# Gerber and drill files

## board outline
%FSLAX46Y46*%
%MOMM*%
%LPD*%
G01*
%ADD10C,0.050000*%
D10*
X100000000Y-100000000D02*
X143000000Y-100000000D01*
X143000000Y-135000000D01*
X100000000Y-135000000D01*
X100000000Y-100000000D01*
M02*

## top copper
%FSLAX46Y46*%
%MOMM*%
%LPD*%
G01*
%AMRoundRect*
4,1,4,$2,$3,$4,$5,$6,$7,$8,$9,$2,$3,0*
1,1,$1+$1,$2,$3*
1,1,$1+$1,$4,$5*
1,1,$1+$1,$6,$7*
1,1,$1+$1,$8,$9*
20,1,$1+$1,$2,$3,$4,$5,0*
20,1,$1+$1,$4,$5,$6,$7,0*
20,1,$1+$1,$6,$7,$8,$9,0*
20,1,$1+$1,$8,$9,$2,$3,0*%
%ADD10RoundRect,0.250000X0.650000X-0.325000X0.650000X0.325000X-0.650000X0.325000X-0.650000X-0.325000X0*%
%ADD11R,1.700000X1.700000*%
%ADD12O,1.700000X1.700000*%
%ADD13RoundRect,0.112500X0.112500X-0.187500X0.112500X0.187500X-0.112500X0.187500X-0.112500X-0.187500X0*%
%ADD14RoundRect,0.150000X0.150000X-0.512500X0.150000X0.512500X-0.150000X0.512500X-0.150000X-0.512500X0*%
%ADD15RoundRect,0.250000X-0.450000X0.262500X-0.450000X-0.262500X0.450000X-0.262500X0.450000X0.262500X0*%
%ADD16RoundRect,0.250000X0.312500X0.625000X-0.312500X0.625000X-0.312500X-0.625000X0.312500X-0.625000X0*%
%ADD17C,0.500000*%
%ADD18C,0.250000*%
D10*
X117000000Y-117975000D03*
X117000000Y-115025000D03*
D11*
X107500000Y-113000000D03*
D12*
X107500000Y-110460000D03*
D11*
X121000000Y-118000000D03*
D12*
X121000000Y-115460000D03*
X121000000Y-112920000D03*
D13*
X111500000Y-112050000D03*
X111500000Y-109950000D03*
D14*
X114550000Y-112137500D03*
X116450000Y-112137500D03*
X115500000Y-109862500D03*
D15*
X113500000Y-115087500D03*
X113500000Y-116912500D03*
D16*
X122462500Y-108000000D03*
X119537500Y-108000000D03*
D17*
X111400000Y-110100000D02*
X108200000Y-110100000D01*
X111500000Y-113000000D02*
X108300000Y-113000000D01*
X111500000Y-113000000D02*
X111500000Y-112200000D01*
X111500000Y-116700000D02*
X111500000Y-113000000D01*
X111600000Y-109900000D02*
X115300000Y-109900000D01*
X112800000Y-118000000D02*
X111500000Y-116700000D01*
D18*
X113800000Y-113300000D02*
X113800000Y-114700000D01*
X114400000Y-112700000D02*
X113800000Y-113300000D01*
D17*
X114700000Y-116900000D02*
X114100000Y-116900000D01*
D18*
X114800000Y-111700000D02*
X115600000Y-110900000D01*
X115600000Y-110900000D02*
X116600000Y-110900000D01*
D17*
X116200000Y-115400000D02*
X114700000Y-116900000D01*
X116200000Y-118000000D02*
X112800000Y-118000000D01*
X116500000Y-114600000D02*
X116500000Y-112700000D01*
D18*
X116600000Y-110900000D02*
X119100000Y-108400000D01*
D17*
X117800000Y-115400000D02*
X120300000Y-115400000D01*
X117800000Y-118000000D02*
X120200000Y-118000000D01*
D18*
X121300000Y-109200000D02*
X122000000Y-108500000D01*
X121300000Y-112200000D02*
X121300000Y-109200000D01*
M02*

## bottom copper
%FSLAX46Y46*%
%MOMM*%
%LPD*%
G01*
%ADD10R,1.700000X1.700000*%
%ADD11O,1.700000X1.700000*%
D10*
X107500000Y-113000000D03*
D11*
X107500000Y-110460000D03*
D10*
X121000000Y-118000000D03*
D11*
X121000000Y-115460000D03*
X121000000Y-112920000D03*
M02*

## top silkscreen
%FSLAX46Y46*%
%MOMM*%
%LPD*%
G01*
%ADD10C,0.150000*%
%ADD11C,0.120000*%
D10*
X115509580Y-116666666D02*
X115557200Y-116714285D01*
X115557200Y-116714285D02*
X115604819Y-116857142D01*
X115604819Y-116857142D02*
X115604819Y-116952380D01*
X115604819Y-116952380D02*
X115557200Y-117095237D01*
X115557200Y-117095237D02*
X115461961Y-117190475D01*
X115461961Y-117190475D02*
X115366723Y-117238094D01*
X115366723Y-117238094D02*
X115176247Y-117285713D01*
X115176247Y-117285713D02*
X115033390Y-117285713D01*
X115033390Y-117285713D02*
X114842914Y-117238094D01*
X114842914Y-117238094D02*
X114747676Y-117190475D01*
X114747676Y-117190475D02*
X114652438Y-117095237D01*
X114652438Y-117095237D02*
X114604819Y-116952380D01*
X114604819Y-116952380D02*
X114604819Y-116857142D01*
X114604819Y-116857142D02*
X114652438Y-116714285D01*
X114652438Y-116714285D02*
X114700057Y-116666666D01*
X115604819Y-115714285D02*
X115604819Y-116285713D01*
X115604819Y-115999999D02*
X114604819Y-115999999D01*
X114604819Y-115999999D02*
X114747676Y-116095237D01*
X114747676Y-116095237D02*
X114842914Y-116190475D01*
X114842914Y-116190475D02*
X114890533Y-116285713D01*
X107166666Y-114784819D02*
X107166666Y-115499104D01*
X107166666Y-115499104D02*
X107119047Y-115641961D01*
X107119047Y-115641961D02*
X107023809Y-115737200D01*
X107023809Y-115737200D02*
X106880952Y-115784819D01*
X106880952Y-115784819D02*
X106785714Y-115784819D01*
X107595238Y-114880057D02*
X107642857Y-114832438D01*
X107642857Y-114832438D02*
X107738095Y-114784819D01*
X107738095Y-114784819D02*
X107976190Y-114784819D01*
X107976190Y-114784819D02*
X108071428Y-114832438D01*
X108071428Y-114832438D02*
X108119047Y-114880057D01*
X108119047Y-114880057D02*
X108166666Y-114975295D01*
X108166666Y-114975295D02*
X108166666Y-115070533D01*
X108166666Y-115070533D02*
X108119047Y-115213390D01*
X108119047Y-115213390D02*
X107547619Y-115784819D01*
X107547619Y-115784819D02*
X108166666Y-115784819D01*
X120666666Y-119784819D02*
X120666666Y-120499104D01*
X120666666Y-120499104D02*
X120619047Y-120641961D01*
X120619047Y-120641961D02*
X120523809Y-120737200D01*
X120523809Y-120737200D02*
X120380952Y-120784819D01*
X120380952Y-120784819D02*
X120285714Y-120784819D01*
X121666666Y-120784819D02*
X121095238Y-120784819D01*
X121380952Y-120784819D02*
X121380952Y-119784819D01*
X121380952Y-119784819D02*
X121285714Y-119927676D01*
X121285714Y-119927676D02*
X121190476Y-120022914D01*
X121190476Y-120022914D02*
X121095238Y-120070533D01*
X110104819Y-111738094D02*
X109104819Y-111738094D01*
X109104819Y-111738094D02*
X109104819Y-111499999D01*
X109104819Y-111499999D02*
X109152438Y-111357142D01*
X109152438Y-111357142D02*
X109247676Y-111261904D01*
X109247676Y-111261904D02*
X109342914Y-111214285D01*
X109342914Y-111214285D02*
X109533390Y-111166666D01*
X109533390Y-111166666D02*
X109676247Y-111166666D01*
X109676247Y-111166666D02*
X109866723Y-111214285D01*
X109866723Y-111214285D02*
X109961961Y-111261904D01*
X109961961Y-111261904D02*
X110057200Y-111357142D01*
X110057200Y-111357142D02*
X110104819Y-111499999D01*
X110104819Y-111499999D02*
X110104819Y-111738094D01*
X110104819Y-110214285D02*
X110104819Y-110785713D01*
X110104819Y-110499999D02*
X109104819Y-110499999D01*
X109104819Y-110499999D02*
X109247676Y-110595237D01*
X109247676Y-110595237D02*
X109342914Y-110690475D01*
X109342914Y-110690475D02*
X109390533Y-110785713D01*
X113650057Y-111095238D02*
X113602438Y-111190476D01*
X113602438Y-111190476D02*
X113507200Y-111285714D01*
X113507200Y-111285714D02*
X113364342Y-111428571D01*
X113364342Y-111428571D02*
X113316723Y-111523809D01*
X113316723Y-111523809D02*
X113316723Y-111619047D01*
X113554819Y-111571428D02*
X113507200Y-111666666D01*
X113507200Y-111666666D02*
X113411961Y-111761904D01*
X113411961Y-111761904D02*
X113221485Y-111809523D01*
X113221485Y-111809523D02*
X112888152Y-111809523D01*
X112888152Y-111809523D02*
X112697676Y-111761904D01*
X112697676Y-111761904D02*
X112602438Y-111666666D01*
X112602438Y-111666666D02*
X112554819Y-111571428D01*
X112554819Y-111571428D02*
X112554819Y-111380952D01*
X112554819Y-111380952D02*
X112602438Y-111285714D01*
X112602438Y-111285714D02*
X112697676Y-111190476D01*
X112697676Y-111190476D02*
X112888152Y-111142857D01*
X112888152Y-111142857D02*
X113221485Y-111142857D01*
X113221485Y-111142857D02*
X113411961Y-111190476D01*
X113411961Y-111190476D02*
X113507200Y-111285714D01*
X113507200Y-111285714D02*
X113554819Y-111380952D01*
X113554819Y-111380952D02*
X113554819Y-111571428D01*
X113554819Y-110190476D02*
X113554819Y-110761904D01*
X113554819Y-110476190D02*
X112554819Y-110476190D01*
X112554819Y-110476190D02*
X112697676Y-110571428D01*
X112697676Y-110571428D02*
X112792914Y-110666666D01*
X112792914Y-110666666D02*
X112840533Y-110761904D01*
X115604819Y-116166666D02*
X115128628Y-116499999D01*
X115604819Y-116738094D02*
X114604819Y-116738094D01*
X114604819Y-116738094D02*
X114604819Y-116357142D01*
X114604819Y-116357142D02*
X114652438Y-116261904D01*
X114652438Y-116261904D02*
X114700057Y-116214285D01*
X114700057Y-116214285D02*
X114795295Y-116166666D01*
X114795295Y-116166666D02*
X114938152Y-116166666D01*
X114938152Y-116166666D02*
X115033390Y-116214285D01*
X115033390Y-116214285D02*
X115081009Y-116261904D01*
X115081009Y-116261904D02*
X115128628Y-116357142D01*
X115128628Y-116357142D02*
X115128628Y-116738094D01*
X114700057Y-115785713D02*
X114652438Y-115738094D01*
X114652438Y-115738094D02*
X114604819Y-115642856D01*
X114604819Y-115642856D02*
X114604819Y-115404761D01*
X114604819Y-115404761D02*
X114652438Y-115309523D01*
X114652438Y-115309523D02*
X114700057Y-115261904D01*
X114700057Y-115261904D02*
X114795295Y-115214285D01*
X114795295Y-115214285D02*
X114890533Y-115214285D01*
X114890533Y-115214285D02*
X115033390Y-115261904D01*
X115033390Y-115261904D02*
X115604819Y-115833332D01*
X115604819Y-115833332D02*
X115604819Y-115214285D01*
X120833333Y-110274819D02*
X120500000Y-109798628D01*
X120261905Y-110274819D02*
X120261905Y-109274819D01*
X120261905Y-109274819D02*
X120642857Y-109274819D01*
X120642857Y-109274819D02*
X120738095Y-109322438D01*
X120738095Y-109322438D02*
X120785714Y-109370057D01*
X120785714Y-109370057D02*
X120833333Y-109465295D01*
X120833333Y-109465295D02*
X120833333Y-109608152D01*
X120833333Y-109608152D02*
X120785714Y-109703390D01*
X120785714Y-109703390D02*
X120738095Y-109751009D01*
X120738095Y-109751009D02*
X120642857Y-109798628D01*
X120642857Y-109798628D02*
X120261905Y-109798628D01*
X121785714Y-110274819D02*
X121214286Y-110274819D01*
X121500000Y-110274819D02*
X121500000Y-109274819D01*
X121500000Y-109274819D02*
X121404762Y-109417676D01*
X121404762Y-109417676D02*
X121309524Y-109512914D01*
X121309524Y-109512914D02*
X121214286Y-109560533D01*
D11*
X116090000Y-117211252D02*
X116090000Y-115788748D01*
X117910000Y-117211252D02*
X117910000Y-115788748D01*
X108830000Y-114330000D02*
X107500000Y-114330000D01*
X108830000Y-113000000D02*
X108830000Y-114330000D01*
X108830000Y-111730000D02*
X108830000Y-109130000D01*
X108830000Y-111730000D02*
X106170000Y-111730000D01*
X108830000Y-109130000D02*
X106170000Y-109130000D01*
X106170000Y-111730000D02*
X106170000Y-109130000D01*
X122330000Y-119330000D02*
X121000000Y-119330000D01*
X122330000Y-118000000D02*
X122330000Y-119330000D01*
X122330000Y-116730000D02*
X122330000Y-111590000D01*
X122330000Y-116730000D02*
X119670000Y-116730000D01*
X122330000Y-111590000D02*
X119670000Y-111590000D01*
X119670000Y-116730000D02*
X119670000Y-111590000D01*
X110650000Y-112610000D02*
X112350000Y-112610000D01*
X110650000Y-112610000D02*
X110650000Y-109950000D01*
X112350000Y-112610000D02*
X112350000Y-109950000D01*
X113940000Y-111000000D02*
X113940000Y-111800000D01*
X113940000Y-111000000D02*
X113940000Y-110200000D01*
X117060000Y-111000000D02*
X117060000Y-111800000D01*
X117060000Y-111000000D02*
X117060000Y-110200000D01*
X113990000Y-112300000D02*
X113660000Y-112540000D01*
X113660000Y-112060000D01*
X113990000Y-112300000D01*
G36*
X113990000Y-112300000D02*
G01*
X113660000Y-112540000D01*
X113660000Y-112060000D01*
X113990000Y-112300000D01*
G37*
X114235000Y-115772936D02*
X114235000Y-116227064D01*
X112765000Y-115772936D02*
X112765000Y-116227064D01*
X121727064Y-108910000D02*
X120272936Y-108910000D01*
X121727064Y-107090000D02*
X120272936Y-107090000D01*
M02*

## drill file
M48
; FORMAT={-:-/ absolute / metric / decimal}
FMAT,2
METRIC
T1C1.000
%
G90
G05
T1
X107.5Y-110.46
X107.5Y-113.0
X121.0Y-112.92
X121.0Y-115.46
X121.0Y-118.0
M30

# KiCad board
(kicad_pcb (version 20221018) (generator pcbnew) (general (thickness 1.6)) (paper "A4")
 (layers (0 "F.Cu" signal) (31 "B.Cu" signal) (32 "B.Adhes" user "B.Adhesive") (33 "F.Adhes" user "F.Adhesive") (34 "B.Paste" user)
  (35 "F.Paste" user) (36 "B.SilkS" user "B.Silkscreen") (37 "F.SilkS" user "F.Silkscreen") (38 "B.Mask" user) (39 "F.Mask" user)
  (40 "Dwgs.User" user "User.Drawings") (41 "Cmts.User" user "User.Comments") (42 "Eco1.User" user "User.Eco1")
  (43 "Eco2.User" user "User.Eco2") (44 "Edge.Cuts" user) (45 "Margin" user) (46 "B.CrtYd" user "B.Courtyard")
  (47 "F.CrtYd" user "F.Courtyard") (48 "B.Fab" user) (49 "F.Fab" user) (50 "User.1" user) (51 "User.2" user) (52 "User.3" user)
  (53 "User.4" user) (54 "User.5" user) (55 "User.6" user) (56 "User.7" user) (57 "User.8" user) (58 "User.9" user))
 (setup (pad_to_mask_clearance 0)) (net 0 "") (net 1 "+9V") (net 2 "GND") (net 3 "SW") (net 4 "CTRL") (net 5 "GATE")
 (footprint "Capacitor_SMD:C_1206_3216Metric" (layer "F.Cu") (at 117 116.5 90)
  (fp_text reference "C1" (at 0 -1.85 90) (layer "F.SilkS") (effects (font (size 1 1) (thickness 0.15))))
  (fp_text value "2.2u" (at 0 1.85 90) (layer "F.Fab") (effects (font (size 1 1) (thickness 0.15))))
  (fp_line (start -0.711252 -0.91) (end 0.711252 -0.91) (stroke (width 0.12) (type solid)) (layer "F.SilkS"))
  (fp_line (start -0.711252 0.91) (end 0.711252 0.91) (stroke (width 0.12) (type solid)) (layer "F.SilkS"))
  (pad "1" smd roundrect (at -1.475 0 90) (size 1.15 1.8) (layers "F.Cu" "F.Paste" "F.Mask") (roundrect_rratio 0.217391) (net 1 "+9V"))
  (pad "2" smd roundrect (at 1.475 0 90) (size 1.15 1.8) (layers "F.Cu" "F.Paste" "F.Mask") (roundrect_rratio 0.217391) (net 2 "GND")))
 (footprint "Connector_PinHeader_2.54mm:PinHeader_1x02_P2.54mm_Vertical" (layer "F.Cu") (at 107.5 113 180)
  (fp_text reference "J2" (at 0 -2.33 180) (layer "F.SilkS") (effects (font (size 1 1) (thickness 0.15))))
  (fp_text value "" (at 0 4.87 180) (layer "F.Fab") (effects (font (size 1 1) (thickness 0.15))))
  (fp_line (start -1.33 -1.33) (end 0 -1.33) (stroke (width 0.12) (type solid)) (layer "F.SilkS"))
  (fp_line (start -1.33 0) (end -1.33 -1.33) (stroke (width 0.12) (type solid)) (layer "F.SilkS"))
  (fp_line (start -1.33 1.27) (end -1.33 3.87) (stroke (width 0.12) (type solid)) (layer "F.SilkS"))
  (fp_line (start -1.33 1.27) (end 1.33 1.27) (stroke (width 0.12) (type solid)) (layer "F.SilkS"))
  (fp_line (start -1.33 3.87) (end 1.33 3.87) (stroke (width 0.12) (type solid)) (layer "F.SilkS"))
  (fp_line (start 1.33 1.27) (end 1.33 3.87) (stroke (width 0.12) (type solid)) (layer "F.SilkS"))
  (pad "1" thru_hole rect (at 0 0 180) (size 1.7 1.7) (drill 1) (layers "*.Cu" "*.Mask") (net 1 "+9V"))
  (pad "2" thru_hole oval (at 0 2.54 180) (size 1.7 1.7) (drill 1) (layers "*.Cu" "*.Mask") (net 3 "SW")))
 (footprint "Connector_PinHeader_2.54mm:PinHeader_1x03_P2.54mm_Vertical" (layer "F.Cu") (at 121 118 180)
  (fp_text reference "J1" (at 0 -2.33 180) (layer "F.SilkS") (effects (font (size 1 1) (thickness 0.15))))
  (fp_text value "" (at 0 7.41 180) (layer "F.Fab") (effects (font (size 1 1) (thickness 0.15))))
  (fp_line (start -1.33 -1.33) (end 0 -1.33) (stroke (width 0.12) (type solid)) (layer "F.SilkS"))
  (fp_line (start -1.33 0) (end -1.33 -1.33) (stroke (width 0.12) (type solid)) (layer "F.SilkS"))
  (fp_line (start -1.33 1.27) (end -1.33 6.41) (stroke (width 0.12) (type solid)) (layer "F.SilkS"))
  (fp_line (start -1.33 1.27) (end 1.33 1.27) (stroke (width 0.12) (type solid)) (layer "F.SilkS"))
  (fp_line (start -1.33 6.41) (end 1.33 6.41) (stroke (width 0.12) (type solid)) (layer "F.SilkS"))
  (fp_line (start 1.33 1.27) (end 1.33 6.41) (stroke (width 0.12) (type solid)) (layer "F.SilkS"))
  (pad "1" thru_hole rect (at 0 0 180) (size 1.7 1.7) (drill 1) (layers "*.Cu" "*.Mask") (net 1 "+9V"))
  (pad "2" thru_hole oval (at 0 2.54 180) (size 1.7 1.7) (drill 1) (layers "*.Cu" "*.Mask") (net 2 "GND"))
  (pad "3" thru_hole oval (at 0 5.08 180) (size 1.7 1.7) (drill 1) (layers "*.Cu" "*.Mask") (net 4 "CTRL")))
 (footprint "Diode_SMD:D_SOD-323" (layer "F.Cu") (at 111.5 111 90)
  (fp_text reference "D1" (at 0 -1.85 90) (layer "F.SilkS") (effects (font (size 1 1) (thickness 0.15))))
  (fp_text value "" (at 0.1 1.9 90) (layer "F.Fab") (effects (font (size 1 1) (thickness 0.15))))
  (fp_line (start -1.61 -0.85) (end -1.61 0.85) (stroke (width 0.12) (type solid)) (layer "F.SilkS"))
  (fp_line (start -1.61 -0.85) (end 1.05 -0.85) (stroke (width 0.12) (type solid)) (layer "F.SilkS"))
  (fp_line (start -1.61 0.85) (end 1.05 0.85) (stroke (width 0.12) (type solid)) (layer "F.SilkS"))
  (pad "1" smd roundrect (at -1.05 0 90) (size 0.6 0.45) (layers "F.Cu" "F.Paste" "F.Mask") (roundrect_rratio 0.25) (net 1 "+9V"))
  (pad "2" smd roundrect (at 1.05 0 90) (size 0.6 0.45) (layers "F.Cu" "F.Paste" "F.Mask") (roundrect_rratio 0.25) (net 3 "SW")))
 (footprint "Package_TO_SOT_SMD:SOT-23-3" (layer "F.Cu") (at 115.5 111 90)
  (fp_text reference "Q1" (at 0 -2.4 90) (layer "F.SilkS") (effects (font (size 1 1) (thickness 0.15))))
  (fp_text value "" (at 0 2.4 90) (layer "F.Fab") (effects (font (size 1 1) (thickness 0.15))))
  (fp_line (start 0 -1.56) (end -0.8 -1.56) (stroke (width 0.12) (type solid)) (layer "F.SilkS"))
  (fp_line (start 0 -1.56) (end 0.8 -1.56) (stroke (width 0.12) (type solid)) (layer "F.SilkS"))
  (fp_line (start 0 1.56) (end -0.8 1.56) (stroke (width 0.12) (type solid)) (layer "F.SilkS"))
  (fp_line (start 0 1.56) (end 0.8 1.56) (stroke (width 0.12) (type solid)) (layer "F.SilkS"))
  (fp_poly
   (pts (xy -1.3 -1.51) (xy -1.54 -1.84) (xy -1.06 -1.84) (xy -1.3 -1.51)) (stroke (width 0.12) (type solid)) (fill solid) (layer "F.SilkS"))
  (pad "1" smd roundrect (at -1.1375 -0.95 90) (size 1.325 0.6) (layers "F.Cu" "F.Paste" "F.Mask") (roundrect_rratio 0.25) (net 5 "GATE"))
  (pad "2" smd roundrect (at -1.1375 0.95 90) (size 1.325 0.6) (layers "F.Cu" "F.Paste" "F.Mask") (roundrect_rratio 0.25) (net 2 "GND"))
  (pad "3" smd roundrect (at 1.1375 0 90) (size 1.325 0.6) (layers "F.Cu" "F.Paste" "F.Mask") (roundrect_rratio 0.25) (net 3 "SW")))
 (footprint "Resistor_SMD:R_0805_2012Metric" (layer "F.Cu") (at 113.5 116 -90)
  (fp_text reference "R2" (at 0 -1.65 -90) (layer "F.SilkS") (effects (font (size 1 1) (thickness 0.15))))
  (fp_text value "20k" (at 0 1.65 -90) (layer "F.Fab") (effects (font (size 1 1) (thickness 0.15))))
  (fp_line (start -0.227064 -0.735) (end 0.227064 -0.735) (stroke (width 0.12) (type solid)) (layer "F.SilkS"))
  (fp_line (start -0.227064 0.735) (end 0.227064 0.735) (stroke (width 0.12) (type solid)) (layer "F.SilkS"))
  (pad "1" smd roundrect (at -0.9125 0 270) (size 1.025 1.4) (layers "F.Cu" "F.Paste" "F.Mask") (roundrect_rratio 0.243902) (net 5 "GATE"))
  (pad "2" smd roundrect (at 0.9125 0 270) (size 1.025 1.4) (layers "F.Cu" "F.Paste" "F.Mask") (roundrect_rratio 0.243902) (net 2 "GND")))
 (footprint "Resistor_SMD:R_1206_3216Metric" (layer "F.Cu") (at 121 108 180)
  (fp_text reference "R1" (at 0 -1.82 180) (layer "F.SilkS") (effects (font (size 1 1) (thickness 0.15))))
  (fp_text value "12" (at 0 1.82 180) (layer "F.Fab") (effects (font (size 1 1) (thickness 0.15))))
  (fp_line (start -0.727064 -0.91) (end 0.727064 -0.91) (stroke (width 0.12) (type solid)) (layer "F.SilkS"))
  (fp_line (start -0.727064 0.91) (end 0.727064 0.91) (stroke (width 0.12) (type solid)) (layer "F.SilkS"))
  (pad "1" smd roundrect (at -1.4625 0 180) (size 1.125 1.75) (layers "F.Cu" "F.Paste" "F.Mask") (roundrect_rratio 0.222222) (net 4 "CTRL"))
  (pad "2" smd roundrect (at 1.4625 0 180) (size 1.125 1.75) (layers "F.Cu" "F.Paste" "F.Mask") (roundrect_rratio 0.222222) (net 5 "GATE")))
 (gr_rect (start 100 100) (end 143 135) (stroke (width 0.05) (type default)) (fill none) (layer "Edge.Cuts"))
 (segment (start 111.4 110.1) (end 108.2 110.1) (width 0.5) (layer "F.Cu") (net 3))
 (segment (start 111.5 113) (end 108.3 113) (width 0.5) (layer "F.Cu") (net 1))
 (segment (start 111.5 113) (end 111.5 112.2) (width 0.5) (layer "F.Cu") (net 1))
 (segment (start 111.5 116.7) (end 111.5 113) (width 0.5) (layer "F.Cu") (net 1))
 (segment (start 111.6 109.9) (end 115.3 109.9) (width 0.5) (layer "F.Cu") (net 3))
 (segment (start 112.8 118) (end 111.5 116.7) (width 0.5) (layer "F.Cu") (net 1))
 (segment (start 113.8 113.3) (end 113.8 114.7) (width 0.25) (layer "F.Cu") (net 5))
 (segment (start 114.4 112.7) (end 113.8 113.3) (width 0.25) (layer "F.Cu") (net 5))
 (segment (start 114.7 116.9) (end 114.1 116.9) (width 0.5) (layer "F.Cu") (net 2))
 (segment (start 114.8 111.7) (end 115.6 110.9) (width 0.25) (layer "F.Cu") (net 5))
 (segment (start 115.6 110.9) (end 116.6 110.9) (width 0.25) (layer "F.Cu") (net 5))
 (segment (start 116.2 115.4) (end 114.7 116.9) (width 0.5) (layer "F.Cu") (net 2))
 (segment (start 116.2 118) (end 112.8 118) (width 0.5) (layer "F.Cu") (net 1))
 (segment (start 116.5 114.6) (end 116.5 112.7) (width 0.5) (layer "F.Cu") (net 2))
 (segment (start 116.6 110.9) (end 119.1 108.4) (width 0.25) (layer "F.Cu") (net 5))
 (segment (start 117.8 115.4) (end 120.3 115.4) (width 0.5) (layer "F.Cu") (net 2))
 (segment (start 117.8 118) (end 120.2 118) (width 0.5) (layer "F.Cu") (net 1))
 (segment (start 121.3 109.2) (end 122 108.5) (width 0.25) (layer "F.Cu") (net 4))
 (segment (start 121.3 112.2) (end 121.3 109.2) (width 0.25) (layer "F.Cu") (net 4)))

